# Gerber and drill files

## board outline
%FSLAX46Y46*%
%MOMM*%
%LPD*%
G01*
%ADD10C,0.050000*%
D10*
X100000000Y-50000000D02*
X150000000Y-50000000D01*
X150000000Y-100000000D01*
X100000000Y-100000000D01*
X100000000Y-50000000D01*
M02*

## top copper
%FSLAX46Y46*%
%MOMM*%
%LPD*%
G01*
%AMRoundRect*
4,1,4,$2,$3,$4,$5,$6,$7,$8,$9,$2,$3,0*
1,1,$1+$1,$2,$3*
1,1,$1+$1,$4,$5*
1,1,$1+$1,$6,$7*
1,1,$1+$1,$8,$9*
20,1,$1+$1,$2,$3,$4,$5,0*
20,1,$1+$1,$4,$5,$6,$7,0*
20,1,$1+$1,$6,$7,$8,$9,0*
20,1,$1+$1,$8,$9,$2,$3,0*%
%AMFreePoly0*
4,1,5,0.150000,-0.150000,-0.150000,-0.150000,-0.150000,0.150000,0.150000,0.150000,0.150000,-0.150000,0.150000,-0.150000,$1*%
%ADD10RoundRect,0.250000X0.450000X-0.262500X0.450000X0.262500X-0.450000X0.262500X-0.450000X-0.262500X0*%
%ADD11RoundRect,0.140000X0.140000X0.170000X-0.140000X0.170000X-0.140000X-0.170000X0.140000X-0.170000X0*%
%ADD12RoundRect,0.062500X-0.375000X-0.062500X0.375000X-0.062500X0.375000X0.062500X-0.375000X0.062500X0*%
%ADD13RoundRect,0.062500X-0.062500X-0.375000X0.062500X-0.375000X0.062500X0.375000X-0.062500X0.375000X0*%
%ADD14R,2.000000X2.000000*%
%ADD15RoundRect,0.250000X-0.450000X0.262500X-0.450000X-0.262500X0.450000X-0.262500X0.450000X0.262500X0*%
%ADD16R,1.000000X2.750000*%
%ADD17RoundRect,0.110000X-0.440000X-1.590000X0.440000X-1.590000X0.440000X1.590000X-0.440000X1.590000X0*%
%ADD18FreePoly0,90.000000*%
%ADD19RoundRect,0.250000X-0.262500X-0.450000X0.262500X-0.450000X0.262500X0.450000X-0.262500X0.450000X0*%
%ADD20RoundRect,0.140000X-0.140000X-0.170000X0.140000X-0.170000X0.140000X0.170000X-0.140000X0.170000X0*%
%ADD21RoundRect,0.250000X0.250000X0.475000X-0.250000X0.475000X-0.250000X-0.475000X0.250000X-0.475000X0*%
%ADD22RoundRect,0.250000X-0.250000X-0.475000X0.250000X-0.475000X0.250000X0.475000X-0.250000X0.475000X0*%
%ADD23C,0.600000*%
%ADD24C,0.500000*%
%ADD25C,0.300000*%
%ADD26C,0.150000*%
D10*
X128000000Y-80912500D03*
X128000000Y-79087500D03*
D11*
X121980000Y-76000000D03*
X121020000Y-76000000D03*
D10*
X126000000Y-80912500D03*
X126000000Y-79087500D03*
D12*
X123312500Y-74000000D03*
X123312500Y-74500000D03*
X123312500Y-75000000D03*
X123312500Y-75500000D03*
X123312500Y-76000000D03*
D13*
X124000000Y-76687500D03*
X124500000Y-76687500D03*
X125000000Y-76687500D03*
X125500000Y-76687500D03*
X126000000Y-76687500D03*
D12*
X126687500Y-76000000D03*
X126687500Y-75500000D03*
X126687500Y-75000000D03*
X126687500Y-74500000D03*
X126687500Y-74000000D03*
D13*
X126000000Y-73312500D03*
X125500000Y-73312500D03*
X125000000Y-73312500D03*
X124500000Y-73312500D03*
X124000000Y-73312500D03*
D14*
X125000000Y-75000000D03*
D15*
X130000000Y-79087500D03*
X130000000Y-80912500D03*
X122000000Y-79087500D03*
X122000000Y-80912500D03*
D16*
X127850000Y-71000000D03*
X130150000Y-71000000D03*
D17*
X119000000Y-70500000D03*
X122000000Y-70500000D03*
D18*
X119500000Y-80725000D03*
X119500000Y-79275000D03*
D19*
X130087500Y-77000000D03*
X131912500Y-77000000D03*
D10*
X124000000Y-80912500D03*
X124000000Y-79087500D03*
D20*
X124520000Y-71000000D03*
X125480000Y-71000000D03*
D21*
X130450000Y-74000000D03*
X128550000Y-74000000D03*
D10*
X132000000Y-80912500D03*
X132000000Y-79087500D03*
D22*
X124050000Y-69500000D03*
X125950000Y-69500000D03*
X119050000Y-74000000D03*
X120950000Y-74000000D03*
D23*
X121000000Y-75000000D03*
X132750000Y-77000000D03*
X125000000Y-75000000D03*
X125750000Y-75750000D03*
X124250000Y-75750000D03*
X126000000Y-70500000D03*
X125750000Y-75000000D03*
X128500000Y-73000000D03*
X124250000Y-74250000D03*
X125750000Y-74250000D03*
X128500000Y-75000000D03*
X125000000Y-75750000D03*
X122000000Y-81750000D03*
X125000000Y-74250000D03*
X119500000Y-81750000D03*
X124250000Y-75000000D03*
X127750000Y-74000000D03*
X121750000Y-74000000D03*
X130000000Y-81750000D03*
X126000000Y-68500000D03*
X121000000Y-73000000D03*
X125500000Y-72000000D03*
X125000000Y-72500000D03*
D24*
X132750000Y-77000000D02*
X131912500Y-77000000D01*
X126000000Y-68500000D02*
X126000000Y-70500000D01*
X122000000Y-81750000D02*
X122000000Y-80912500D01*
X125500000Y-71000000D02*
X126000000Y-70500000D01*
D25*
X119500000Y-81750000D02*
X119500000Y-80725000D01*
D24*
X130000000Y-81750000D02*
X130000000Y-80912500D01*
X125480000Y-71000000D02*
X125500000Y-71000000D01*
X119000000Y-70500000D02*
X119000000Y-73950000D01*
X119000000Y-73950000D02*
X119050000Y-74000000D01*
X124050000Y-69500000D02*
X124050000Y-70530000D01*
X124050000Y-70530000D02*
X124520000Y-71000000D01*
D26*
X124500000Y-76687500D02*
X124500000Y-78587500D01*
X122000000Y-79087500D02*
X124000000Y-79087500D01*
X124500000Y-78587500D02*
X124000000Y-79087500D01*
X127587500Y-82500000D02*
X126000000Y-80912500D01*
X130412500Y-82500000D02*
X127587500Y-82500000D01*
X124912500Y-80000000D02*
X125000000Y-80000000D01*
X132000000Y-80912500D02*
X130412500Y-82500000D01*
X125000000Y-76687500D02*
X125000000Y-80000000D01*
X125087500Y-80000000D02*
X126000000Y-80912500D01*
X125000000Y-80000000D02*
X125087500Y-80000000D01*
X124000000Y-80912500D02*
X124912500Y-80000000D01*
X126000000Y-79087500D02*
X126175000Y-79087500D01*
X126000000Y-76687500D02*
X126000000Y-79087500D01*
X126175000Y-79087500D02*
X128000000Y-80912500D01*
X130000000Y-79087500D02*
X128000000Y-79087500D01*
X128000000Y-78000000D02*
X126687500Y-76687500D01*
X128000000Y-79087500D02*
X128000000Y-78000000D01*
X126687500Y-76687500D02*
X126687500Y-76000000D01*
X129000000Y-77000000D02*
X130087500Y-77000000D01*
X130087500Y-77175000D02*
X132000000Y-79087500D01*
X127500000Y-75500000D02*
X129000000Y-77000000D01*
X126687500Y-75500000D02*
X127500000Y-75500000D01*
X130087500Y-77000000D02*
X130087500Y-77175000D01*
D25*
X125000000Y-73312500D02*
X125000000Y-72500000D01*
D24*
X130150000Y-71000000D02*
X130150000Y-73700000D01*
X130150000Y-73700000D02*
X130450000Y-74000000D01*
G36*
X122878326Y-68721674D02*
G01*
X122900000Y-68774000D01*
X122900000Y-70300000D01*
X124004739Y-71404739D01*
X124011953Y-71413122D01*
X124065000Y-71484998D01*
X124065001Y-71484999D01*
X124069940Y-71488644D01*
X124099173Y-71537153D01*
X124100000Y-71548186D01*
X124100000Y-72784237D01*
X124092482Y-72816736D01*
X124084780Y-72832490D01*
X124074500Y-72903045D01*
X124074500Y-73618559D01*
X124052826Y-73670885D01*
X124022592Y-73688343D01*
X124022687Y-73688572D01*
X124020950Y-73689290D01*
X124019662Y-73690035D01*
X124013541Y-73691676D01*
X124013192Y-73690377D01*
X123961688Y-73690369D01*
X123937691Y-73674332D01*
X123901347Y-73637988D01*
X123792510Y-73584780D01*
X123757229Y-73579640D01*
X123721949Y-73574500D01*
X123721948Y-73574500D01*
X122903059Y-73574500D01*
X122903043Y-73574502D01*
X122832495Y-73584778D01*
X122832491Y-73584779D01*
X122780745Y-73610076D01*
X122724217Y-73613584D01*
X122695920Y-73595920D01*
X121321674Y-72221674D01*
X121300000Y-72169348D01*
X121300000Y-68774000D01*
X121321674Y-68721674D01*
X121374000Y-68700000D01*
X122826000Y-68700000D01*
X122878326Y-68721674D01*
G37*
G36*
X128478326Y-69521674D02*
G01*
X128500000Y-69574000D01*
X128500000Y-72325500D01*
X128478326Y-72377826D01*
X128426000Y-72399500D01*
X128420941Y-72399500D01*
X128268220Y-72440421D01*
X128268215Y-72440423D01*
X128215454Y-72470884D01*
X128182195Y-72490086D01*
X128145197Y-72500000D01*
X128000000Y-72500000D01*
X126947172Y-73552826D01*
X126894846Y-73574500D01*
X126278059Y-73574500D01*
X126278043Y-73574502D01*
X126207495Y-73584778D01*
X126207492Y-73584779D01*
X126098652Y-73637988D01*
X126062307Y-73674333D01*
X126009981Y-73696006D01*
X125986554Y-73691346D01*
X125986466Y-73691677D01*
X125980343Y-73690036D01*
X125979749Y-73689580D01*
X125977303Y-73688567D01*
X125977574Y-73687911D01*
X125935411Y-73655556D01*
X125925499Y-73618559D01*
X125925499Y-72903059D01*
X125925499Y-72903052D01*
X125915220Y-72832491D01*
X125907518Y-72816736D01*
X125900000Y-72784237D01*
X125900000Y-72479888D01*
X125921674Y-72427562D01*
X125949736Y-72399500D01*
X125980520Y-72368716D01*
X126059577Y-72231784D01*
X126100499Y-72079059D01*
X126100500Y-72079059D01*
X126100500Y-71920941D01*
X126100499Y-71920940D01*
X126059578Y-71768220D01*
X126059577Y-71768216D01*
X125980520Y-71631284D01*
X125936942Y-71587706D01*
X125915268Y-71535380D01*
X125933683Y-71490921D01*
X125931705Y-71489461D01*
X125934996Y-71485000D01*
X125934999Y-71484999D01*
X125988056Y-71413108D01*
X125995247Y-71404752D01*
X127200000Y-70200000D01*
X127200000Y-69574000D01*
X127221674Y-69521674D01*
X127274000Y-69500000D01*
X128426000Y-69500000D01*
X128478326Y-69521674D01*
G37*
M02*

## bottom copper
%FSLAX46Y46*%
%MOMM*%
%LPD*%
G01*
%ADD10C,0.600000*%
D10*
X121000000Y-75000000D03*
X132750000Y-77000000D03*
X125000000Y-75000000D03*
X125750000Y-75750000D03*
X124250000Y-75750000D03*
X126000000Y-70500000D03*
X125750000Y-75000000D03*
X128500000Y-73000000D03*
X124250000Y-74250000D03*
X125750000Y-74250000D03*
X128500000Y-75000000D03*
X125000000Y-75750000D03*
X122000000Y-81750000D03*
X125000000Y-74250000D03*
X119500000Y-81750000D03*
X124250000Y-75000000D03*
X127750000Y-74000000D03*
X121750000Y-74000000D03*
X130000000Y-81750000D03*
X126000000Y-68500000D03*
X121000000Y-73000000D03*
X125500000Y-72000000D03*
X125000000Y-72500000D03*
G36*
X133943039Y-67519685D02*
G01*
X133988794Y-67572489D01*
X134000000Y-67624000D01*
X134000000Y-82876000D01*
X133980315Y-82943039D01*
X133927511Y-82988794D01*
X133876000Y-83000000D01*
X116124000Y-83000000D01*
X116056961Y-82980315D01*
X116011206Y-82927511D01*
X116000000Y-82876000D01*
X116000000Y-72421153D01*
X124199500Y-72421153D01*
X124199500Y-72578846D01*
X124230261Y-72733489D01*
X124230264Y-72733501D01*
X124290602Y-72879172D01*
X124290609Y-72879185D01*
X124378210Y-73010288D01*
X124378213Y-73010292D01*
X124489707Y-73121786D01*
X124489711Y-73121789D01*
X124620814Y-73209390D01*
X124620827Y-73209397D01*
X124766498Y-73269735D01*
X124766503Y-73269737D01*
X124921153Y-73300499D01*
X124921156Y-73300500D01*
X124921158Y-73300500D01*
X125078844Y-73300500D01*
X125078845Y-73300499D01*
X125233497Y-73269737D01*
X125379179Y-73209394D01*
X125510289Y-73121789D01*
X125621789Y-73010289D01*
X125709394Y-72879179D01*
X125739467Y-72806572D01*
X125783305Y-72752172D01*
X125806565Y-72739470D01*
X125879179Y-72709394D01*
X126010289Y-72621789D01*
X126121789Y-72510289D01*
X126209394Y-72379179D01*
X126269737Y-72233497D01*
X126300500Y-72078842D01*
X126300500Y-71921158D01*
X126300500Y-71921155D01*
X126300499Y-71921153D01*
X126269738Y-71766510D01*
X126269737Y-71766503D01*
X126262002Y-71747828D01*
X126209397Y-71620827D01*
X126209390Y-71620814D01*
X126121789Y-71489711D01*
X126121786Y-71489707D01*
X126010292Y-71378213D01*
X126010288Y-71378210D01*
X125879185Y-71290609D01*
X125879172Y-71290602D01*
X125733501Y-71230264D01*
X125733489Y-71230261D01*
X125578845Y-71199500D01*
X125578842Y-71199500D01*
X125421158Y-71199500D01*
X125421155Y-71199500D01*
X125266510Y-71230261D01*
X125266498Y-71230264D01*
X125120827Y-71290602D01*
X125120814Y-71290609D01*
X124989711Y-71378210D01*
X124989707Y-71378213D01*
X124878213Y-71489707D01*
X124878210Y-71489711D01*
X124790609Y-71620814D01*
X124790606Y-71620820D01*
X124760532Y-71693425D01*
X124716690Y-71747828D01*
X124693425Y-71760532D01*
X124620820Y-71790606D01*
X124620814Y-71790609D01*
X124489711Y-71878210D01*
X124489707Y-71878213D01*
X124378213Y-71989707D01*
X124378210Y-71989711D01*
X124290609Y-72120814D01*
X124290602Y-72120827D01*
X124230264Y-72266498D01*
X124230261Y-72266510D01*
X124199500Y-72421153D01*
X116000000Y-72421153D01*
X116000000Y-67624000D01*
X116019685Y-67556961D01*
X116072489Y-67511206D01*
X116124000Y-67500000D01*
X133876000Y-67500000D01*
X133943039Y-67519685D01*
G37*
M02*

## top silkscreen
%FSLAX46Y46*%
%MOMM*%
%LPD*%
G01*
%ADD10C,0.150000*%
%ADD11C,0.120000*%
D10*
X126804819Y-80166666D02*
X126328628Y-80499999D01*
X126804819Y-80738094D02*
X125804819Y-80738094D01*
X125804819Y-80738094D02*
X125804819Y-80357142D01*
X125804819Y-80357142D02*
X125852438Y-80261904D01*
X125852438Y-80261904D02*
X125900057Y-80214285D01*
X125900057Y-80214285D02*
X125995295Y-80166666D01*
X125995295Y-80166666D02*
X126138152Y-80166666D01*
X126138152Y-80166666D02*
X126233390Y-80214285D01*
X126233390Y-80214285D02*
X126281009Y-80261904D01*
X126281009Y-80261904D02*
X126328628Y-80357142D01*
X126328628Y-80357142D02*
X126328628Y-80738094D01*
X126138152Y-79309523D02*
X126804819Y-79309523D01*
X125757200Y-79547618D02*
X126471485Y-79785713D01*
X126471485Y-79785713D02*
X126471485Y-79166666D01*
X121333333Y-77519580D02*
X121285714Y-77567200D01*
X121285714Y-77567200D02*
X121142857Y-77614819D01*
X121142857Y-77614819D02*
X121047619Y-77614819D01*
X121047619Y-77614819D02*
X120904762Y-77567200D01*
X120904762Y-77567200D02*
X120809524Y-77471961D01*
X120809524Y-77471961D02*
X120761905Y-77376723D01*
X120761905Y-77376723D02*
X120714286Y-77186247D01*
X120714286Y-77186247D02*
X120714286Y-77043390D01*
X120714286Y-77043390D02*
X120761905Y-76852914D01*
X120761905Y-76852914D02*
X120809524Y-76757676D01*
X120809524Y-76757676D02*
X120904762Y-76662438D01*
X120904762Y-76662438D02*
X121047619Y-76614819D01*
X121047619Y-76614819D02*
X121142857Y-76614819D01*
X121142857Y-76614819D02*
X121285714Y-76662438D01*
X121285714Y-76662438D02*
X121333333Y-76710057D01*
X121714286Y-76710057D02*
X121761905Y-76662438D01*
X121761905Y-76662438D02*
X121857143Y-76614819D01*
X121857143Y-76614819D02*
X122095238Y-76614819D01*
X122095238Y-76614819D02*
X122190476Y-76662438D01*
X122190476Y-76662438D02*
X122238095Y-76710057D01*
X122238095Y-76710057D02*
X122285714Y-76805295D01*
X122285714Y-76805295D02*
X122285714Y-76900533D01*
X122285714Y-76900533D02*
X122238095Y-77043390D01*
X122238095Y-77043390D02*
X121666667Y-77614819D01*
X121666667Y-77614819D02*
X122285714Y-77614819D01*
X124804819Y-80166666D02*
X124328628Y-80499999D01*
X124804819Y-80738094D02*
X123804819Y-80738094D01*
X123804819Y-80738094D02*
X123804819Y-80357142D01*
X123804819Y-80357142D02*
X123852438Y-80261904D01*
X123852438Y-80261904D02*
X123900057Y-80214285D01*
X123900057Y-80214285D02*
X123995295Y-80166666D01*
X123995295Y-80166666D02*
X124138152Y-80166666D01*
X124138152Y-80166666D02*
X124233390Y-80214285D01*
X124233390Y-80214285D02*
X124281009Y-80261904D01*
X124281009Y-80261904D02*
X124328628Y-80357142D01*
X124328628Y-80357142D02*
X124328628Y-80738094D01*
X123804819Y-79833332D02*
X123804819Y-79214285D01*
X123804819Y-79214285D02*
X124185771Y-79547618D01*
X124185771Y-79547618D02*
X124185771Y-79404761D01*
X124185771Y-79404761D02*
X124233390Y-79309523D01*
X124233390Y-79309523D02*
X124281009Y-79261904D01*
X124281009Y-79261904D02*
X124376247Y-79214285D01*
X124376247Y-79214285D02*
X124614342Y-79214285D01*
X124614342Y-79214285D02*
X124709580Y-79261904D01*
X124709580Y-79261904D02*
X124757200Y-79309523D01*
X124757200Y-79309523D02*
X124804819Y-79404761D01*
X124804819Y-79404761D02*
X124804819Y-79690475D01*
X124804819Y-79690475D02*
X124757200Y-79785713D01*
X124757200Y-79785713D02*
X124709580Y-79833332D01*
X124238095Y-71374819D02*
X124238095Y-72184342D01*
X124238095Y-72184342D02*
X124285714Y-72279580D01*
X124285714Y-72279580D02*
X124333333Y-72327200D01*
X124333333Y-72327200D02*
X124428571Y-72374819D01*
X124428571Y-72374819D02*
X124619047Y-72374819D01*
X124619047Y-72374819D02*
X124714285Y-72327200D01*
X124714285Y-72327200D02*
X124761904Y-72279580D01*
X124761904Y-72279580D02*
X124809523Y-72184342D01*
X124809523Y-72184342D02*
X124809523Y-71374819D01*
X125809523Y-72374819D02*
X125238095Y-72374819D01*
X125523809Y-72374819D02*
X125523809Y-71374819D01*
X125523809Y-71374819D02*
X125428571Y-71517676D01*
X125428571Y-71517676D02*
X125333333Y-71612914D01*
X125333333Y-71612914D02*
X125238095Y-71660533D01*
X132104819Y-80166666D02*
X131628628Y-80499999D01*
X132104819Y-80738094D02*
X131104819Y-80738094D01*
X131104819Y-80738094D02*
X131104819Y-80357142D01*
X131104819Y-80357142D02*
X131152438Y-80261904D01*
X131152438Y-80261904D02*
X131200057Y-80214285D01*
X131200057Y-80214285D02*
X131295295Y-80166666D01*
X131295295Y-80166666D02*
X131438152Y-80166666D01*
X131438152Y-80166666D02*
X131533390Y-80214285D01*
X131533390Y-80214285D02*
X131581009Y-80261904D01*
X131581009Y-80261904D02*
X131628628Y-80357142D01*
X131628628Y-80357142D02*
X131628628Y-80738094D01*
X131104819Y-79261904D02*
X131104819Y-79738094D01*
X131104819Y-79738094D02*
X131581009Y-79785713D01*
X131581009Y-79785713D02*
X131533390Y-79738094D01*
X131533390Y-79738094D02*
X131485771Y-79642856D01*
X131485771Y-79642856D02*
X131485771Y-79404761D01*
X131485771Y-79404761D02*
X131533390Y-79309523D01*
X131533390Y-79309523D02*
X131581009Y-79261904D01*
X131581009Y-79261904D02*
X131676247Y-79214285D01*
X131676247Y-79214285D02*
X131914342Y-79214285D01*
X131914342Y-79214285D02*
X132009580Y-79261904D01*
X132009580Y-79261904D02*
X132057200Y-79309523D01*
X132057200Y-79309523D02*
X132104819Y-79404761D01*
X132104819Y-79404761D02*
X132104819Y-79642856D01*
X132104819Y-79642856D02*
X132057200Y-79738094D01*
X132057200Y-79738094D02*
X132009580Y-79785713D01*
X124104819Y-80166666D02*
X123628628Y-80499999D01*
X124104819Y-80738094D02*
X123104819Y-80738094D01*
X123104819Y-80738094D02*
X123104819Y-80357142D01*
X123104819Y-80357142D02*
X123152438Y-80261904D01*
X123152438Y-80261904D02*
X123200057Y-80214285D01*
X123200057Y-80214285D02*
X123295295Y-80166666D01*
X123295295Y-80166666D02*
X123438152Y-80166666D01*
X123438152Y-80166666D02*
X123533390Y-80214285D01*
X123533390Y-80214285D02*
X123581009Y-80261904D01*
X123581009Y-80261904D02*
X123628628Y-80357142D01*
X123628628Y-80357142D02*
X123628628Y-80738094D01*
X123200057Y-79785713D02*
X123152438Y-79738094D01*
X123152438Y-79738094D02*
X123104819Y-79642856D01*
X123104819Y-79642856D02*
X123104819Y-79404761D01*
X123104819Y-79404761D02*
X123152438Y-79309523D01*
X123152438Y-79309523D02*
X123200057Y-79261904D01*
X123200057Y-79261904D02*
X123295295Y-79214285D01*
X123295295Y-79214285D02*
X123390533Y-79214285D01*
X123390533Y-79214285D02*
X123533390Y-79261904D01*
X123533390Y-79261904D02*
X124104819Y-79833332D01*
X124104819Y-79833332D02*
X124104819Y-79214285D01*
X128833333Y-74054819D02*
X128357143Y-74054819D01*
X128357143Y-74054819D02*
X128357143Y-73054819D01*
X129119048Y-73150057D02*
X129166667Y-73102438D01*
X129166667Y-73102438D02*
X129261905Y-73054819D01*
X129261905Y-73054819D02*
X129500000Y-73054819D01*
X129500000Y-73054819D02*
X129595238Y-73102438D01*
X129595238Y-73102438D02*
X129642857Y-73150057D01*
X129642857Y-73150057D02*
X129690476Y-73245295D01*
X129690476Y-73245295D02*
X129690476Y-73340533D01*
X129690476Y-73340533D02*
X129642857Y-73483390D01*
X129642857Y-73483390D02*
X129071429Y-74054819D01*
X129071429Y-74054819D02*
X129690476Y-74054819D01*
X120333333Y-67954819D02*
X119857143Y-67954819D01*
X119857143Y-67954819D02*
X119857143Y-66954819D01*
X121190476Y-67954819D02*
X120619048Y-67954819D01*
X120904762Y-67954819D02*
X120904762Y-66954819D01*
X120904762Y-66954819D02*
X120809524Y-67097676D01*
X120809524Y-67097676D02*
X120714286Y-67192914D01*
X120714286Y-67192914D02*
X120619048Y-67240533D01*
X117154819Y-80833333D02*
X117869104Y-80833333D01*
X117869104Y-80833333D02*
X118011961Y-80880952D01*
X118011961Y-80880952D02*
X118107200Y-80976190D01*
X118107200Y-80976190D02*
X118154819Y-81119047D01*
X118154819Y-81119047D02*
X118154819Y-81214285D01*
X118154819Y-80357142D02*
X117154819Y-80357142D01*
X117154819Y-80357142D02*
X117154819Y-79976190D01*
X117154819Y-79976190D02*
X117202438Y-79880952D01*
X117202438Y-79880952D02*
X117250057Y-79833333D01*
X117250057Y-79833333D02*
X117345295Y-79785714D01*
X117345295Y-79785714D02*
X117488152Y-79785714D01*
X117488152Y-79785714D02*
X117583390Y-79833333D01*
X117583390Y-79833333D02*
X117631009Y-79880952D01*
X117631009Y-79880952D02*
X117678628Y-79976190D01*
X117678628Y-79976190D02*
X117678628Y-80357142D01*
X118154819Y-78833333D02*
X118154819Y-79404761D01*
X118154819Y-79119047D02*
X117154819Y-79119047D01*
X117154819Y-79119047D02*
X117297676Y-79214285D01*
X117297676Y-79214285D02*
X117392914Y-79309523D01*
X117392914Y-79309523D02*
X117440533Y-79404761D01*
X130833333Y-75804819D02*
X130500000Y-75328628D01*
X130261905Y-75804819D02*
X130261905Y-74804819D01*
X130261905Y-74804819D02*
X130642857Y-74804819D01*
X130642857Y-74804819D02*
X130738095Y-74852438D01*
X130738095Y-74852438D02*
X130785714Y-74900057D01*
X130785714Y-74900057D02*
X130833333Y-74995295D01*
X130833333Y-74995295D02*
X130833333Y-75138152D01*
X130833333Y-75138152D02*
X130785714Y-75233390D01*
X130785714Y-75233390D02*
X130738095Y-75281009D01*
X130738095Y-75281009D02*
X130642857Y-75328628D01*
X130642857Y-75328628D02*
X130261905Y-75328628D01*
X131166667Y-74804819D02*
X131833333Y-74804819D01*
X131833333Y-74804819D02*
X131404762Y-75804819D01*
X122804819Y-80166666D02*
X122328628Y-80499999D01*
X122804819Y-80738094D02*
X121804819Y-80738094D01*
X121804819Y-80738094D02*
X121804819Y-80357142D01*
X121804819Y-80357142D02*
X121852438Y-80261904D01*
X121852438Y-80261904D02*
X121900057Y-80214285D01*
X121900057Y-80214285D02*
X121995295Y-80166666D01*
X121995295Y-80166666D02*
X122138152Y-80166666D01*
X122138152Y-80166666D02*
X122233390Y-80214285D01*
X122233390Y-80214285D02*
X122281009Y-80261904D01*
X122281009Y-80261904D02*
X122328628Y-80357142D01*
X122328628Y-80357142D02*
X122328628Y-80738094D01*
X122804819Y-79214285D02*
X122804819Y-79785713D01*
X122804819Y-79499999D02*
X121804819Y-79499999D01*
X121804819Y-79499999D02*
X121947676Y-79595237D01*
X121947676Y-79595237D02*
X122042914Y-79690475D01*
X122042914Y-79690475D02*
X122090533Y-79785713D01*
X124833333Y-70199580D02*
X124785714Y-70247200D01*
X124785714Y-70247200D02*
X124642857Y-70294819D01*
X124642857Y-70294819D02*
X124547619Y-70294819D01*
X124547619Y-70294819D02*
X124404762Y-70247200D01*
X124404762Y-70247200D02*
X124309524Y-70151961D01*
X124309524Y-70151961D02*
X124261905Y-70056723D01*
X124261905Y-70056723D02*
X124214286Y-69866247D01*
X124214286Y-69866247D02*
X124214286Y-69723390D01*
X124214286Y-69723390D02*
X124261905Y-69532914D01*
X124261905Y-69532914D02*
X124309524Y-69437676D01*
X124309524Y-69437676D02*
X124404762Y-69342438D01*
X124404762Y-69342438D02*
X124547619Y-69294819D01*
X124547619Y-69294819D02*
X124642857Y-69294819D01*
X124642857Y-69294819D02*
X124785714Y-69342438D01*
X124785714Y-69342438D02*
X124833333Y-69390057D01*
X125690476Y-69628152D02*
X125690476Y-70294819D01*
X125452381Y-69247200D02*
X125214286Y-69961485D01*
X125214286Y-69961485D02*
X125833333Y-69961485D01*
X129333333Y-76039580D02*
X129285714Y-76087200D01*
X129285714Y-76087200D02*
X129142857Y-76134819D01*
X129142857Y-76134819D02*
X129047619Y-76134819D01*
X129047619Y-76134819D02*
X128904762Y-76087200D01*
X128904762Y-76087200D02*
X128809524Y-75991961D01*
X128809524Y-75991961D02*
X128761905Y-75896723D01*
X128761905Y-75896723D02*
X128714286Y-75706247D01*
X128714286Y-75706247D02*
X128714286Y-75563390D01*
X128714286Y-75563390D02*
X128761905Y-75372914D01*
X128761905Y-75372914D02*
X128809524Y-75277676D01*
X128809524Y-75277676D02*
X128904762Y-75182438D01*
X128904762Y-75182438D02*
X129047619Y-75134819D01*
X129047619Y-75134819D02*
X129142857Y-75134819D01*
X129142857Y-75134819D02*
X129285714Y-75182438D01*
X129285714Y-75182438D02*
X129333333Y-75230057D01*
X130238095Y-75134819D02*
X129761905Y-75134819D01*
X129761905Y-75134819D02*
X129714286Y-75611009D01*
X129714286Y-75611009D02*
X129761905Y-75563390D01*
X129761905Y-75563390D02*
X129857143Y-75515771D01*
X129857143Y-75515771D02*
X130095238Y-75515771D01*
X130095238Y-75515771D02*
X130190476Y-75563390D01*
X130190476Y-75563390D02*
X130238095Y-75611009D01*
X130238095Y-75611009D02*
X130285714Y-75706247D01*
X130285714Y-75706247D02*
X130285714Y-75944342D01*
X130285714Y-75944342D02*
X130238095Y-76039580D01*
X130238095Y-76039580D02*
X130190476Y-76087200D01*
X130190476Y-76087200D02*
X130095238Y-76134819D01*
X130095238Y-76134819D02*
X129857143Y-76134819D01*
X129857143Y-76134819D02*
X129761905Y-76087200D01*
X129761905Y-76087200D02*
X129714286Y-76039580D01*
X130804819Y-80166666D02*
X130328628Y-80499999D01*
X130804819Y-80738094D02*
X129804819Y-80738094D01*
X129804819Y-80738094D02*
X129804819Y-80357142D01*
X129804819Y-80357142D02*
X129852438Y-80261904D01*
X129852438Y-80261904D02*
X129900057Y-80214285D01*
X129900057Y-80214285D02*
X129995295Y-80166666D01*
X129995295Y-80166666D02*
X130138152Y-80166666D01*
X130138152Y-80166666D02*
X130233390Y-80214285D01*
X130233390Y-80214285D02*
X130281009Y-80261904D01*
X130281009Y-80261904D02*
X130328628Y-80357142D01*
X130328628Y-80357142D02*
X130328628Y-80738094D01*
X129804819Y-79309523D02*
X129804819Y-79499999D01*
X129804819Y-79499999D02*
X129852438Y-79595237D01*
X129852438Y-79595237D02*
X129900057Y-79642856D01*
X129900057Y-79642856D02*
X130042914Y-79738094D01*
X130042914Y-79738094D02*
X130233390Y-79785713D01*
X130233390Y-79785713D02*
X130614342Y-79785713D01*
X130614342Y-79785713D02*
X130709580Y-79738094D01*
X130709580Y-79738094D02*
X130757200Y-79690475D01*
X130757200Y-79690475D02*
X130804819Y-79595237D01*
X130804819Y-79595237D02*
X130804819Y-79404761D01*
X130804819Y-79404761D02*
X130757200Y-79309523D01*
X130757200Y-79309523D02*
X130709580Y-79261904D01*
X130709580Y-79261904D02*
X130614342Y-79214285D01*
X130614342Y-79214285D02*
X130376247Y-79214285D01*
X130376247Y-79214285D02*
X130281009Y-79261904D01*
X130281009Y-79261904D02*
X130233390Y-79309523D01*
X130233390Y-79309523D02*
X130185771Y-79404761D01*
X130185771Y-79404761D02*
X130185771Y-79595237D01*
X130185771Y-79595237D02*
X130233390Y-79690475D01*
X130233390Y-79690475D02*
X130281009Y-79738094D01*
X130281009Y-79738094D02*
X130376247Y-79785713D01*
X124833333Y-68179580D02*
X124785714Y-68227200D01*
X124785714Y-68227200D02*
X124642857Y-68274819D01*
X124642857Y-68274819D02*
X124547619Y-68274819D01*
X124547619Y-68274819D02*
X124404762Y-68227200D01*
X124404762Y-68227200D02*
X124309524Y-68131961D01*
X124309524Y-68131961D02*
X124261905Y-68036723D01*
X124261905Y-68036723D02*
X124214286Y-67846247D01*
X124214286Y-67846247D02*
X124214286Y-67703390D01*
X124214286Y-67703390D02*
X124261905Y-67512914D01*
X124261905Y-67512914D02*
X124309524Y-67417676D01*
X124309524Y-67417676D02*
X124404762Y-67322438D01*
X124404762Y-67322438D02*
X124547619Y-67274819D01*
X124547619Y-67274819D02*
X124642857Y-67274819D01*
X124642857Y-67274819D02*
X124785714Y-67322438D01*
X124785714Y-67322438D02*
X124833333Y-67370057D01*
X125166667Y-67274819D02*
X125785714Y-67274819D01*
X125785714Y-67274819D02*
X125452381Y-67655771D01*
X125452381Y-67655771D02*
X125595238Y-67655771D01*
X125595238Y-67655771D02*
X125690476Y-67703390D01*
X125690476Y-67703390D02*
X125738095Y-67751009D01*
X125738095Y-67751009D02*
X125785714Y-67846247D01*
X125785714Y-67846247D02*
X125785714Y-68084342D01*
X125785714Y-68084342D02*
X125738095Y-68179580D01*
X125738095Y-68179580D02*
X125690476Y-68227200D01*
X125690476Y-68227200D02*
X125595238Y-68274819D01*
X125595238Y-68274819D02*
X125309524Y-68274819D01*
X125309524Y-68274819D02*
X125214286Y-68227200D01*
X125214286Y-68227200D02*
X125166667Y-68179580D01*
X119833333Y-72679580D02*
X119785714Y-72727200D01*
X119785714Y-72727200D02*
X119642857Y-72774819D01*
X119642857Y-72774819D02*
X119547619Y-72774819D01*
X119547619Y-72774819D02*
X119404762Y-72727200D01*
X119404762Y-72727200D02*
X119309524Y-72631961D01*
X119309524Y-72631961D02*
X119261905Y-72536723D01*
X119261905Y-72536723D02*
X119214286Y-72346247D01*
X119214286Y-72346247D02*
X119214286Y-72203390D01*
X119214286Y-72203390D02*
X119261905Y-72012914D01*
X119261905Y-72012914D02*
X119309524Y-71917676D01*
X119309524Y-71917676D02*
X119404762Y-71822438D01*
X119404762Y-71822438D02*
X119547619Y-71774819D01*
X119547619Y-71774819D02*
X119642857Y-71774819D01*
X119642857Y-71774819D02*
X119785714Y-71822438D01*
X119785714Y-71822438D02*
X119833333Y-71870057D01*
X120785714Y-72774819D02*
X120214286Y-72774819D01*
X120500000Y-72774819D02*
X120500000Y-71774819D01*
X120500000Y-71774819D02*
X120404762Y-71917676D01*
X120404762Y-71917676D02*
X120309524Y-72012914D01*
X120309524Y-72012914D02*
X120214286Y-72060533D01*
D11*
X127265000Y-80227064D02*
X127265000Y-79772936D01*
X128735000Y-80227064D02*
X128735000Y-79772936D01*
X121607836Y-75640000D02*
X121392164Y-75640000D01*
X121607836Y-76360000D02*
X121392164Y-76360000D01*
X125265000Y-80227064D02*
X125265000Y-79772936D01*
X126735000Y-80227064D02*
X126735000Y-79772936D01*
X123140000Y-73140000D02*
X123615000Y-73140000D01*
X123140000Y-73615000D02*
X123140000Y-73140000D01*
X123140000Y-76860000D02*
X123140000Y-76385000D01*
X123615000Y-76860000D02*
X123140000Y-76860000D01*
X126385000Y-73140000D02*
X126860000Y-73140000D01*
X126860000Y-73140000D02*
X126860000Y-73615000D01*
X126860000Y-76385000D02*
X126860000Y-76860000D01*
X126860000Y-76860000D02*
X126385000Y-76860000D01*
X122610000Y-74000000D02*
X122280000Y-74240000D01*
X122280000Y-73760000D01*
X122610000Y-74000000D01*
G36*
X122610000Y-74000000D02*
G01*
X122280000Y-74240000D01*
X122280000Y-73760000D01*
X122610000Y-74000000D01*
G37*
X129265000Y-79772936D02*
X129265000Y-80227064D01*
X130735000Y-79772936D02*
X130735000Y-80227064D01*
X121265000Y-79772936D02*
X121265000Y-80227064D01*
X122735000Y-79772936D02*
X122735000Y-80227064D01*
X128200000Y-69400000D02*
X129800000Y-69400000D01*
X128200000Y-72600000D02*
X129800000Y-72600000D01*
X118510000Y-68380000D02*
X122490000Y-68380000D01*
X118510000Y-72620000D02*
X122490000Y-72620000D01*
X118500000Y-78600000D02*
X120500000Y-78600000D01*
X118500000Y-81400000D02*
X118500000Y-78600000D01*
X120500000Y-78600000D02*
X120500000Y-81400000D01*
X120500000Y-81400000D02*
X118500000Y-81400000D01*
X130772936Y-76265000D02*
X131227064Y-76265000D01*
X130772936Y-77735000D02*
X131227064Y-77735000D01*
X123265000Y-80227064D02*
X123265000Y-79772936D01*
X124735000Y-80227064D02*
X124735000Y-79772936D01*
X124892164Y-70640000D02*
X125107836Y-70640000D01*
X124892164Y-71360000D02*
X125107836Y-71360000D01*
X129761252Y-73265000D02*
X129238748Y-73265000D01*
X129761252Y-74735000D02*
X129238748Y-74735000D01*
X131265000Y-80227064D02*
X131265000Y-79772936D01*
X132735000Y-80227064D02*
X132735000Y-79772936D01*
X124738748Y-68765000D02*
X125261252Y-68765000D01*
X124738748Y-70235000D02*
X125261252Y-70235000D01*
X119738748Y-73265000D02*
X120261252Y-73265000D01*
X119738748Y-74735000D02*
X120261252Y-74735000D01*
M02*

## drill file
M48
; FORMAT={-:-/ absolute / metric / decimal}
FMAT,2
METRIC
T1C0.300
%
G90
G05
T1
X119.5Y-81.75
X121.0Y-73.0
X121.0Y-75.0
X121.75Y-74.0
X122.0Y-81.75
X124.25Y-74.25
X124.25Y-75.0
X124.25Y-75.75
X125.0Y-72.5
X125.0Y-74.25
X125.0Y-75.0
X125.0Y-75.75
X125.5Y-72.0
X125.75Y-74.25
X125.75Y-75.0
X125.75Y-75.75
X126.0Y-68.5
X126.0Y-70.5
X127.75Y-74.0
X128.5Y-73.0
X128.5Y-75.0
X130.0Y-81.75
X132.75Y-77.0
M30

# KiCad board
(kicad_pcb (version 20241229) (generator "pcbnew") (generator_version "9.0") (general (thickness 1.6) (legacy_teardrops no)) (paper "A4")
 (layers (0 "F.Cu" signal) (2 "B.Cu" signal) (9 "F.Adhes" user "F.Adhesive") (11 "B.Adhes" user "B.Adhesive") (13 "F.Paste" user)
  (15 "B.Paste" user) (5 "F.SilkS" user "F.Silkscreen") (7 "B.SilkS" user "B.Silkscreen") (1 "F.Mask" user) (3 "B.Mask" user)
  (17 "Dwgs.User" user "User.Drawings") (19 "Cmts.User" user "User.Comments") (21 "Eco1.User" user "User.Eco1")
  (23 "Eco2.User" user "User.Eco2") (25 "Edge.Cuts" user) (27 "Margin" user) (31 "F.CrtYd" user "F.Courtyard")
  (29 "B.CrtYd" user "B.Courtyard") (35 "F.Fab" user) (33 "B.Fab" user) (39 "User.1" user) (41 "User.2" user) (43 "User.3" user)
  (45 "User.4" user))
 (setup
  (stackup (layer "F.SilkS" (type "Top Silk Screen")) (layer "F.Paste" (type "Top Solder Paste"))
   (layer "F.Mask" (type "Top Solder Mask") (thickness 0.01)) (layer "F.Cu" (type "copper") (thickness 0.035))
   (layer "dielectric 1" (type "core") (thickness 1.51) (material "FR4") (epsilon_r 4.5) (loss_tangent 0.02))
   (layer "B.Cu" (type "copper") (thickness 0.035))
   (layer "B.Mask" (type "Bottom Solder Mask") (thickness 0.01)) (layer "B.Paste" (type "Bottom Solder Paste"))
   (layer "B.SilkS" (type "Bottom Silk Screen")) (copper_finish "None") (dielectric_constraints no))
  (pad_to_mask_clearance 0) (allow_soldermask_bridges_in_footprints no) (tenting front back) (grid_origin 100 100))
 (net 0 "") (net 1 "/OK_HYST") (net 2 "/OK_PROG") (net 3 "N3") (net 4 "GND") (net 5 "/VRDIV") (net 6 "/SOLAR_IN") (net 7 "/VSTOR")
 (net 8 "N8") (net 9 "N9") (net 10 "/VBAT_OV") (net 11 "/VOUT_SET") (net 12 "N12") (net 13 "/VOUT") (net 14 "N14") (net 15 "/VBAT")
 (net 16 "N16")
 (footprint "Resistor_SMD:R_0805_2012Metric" (layer "F.Cu") (at 128 80 90)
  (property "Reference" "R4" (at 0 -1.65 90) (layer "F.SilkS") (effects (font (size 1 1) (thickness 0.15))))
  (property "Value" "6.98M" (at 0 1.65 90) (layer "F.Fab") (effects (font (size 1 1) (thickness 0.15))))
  (fp_line (start -0.227064 -0.735) (end 0.227064 -0.735) (stroke (width 0.12) (type solid)) (layer "F.SilkS"))
  (fp_line (start -0.227064 0.735) (end 0.227064 0.735) (stroke (width 0.12) (type solid)) (layer "F.SilkS"))
  (pad "1" smd roundrect (at -0.9125 0 90) (size 1.025 1.4) (layers "F.Cu" "F.Mask" "F.Paste") (roundrect_rratio 0.243902)
   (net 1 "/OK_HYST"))
  (pad "2" smd roundrect (at 0.9125 0 90) (size 1.025 1.4) (layers "F.Cu" "F.Mask" "F.Paste") (roundrect_rratio 0.243902) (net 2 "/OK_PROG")))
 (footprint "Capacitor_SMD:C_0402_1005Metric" (layer "F.Cu") (at 121.5 76 180)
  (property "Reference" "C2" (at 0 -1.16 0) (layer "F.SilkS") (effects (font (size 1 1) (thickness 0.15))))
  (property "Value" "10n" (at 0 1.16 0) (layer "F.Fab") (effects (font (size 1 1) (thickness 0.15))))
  (fp_line (start -0.107836 0.36) (end 0.107836 0.36) (stroke (width 0.12) (type solid)) (layer "F.SilkS"))
  (fp_line (start -0.107836 -0.36) (end 0.107836 -0.36) (stroke (width 0.12) (type solid)) (layer "F.SilkS"))
  (pad "1" smd roundrect (at -0.48 0 180) (size 0.56 0.62) (layers "F.Cu" "F.Mask" "F.Paste") (roundrect_rratio 0.25) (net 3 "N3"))
  (pad "2" smd roundrect (at 0.48 0 180) (size 0.56 0.62) (layers "F.Cu" "F.Mask" "F.Paste") (roundrect_rratio 0.25) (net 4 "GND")))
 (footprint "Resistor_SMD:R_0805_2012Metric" (layer "F.Cu") (at 126 80 90)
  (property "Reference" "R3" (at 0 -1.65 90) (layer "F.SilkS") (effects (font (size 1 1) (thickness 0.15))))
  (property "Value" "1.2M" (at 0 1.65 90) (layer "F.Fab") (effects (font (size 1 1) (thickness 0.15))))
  (fp_line (start -0.227064 -0.735) (end 0.227064 -0.735) (stroke (width 0.12) (type solid)) (layer "F.SilkS"))
  (fp_line (start -0.227064 0.735) (end 0.227064 0.735) (stroke (width 0.12) (type solid)) (layer "F.SilkS"))
  (pad "1" smd roundrect (at -0.9125 0 90) (size 1.025 1.4) (layers "F.Cu" "F.Mask" "F.Paste") (roundrect_rratio 0.243902) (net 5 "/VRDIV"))
  (pad "2" smd roundrect (at 0.9125 0 90) (size 1.025 1.4) (layers "F.Cu" "F.Mask" "F.Paste") (roundrect_rratio 0.243902) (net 1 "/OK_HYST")))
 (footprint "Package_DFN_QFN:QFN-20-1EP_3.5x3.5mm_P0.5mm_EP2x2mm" (layer "F.Cu") (at 125 75)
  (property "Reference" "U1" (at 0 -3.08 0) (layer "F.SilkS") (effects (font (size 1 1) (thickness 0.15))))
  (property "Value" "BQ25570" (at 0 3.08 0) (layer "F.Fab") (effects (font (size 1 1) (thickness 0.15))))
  (fp_line (start -1.86 -1.86) (end -1.385 -1.86) (stroke (width 0.12) (type solid)) (layer "F.SilkS"))
  (fp_line (start -1.86 -1.385) (end -1.86 -1.86) (stroke (width 0.12) (type solid)) (layer "F.SilkS"))
  (fp_line (start -1.86 1.86) (end -1.86 1.385) (stroke (width 0.12) (type solid)) (layer "F.SilkS"))
  (fp_line (start -1.385 1.86) (end -1.86 1.86) (stroke (width 0.12) (type solid)) (layer "F.SilkS"))
  (fp_line (start 1.385 -1.86) (end 1.86 -1.86) (stroke (width 0.12) (type solid)) (layer "F.SilkS"))
  (fp_line (start 1.86 -1.86) (end 1.86 -1.385) (stroke (width 0.12) (type solid)) (layer "F.SilkS"))
  (fp_line (start 1.86 1.385) (end 1.86 1.86) (stroke (width 0.12) (type solid)) (layer "F.SilkS"))
  (fp_line (start 1.86 1.86) (end 1.385 1.86) (stroke (width 0.12) (type solid)) (layer "F.SilkS"))
  (fp_poly (pts (xy -2.39 -1) (xy -2.72 -0.76) (xy -2.72 -1.24)) (stroke (width 0.12) (type solid)) (fill yes) (layer "F.SilkS"))
  (pad "" smd roundrect (at -0.5 -0.5) (size 0.81 0.81) (layers "F.Paste") (roundrect_rratio 0.25))
  (pad "" smd roundrect (at -0.5 0.5) (size 0.81 0.81) (layers "F.Paste") (roundrect_rratio 0.25))
  (pad "" smd roundrect (at 0.5 -0.5) (size 0.81 0.81) (layers "F.Paste") (roundrect_rratio 0.25))
  (pad "" smd roundrect (at 0.5 0.5) (size 0.81 0.81) (layers "F.Paste") (roundrect_rratio 0.25))
  (pad "1" smd roundrect (at -1.6875 -1) (size 0.875 0.25) (layers "F.Cu" "F.Mask" "F.Paste") (roundrect_rratio 0.25) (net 4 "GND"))
  (pad "2" smd roundrect (at -1.6875 -0.5) (size 0.875 0.25) (layers "F.Cu" "F.Mask" "F.Paste") (roundrect_rratio 0.25) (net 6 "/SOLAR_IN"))
  (pad "3" smd roundrect (at -1.6875 0) (size 0.875 0.25) (layers "F.Cu" "F.Mask" "F.Paste") (roundrect_rratio 0.25) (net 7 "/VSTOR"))
  (pad "4" smd roundrect (at -1.6875 0.5) (size 0.875 0.25) (layers "F.Cu" "F.Mask" "F.Paste") (roundrect_rratio 0.25) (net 3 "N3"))
  (pad "5" smd roundrect (at -1.6875 1) (size 0.875 0.25) (layers "F.Cu" "F.Mask" "F.Paste") (roundrect_rratio 0.25) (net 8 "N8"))
  (pad "6" smd roundrect (at -1 1.6875) (size 0.25 0.875) (layers "F.Cu" "F.Mask" "F.Paste") (roundrect_rratio 0.25) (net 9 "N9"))
  (pad "7" smd roundrect (at -0.5 1.6875) (size 0.25 0.875) (layers "F.Cu" "F.Mask" "F.Paste") (roundrect_rratio 0.25) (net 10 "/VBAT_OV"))
  (pad "8" smd roundrect (at 0 1.6875) (size 0.25 0.875) (layers "F.Cu" "F.Mask" "F.Paste") (roundrect_rratio 0.25) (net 5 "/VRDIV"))
  (pad "9" smd roundrect (at 0.5 1.6875) (size 0.25 0.875) (layers "F.Cu" "F.Mask" "F.Paste") (roundrect_rratio 0.25) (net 4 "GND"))
  (pad "10" smd roundrect (at 1 1.6875) (size 0.25 0.875) (layers "F.Cu" "F.Mask" "F.Paste") (roundrect_rratio 0.25) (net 1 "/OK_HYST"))
  (pad "11" smd roundrect (at 1.6875 1) (size 0.875 0.25) (layers "F.Cu" "F.Mask" "F.Paste") (roundrect_rratio 0.25) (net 2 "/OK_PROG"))
  (pad "12" smd roundrect (at 1.6875 0.5) (size 0.875 0.25) (layers "F.Cu" "F.Mask" "F.Paste") (roundrect_rratio 0.25) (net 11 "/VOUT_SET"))
  (pad "13" smd roundrect (at 1.6875 0) (size 0.875 0.25) (layers "F.Cu" "F.Mask" "F.Paste") (roundrect_rratio 0.25) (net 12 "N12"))
  (pad "14" smd roundrect (at 1.6875 -0.5) (size 0.875 0.25) (layers "F.Cu" "F.Mask" "F.Paste") (roundrect_rratio 0.25) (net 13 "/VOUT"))
  (pad "15" smd roundrect (at 1.6875 -1) (size 0.875 0.25) (layers "F.Cu" "F.Mask" "F.Paste") (roundrect_rratio 0.25) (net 4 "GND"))
  (pad "16" smd roundrect (at 1 -1.6875) (size 0.25 0.875) (layers "F.Cu" "F.Mask" "F.Paste") (roundrect_rratio 0.25) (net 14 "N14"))
  (pad "17" smd roundrect (at 0.5 -1.6875) (size 0.25 0.875) (layers "F.Cu" "F.Mask" "F.Paste") (roundrect_rratio 0.25) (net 4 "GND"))
  (pad "18" smd roundrect (at 0 -1.6875) (size 0.25 0.875) (layers "F.Cu" "F.Mask" "F.Paste") (roundrect_rratio 0.25) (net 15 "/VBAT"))
  (pad "19" smd roundrect (at -0.5 -1.6875) (size 0.25 0.875) (layers "F.Cu" "F.Mask" "F.Paste") (roundrect_rratio 0.25) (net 7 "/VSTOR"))
  (pad "20" smd roundrect (at -1 -1.6875) (size 0.25 0.875) (layers "F.Cu" "F.Mask" "F.Paste") (roundrect_rratio 0.25) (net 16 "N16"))
  (pad "21" smd rect (at 0 0) (size 2 2) (layers "F.Cu" "F.Mask") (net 4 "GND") (zone_connect 2)))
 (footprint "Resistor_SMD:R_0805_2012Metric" (layer "F.Cu") (at 130 80 -90)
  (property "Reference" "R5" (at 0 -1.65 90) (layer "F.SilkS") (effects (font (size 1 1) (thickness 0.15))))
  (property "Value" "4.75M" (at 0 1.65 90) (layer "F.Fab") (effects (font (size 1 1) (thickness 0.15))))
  (fp_line (start -0.227064 0.735) (end 0.227064 0.735) (stroke (width 0.12) (type solid)) (layer "F.SilkS"))
  (fp_line (start -0.227064 -0.735) (end 0.227064 -0.735) (stroke (width 0.12) (type solid)) (layer "F.SilkS"))
  (pad "1" smd roundrect (at -0.9125 0 270) (size 1.025 1.4) (layers "F.Cu" "F.Mask" "F.Paste") (roundrect_rratio 0.243902)
   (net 2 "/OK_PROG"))
  (pad "2" smd roundrect (at 0.9125 0 270) (size 1.025 1.4) (layers "F.Cu" "F.Mask" "F.Paste") (roundrect_rratio 0.243902) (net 4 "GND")))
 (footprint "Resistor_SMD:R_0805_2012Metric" (layer "F.Cu") (at 122 80 -90)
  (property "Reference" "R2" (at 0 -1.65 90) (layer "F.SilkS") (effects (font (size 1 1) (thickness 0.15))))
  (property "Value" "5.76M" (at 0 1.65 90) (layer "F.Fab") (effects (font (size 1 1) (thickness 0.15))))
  (fp_line (start -0.227064 0.735) (end 0.227064 0.735) (stroke (width 0.12) (type solid)) (layer "F.SilkS"))
  (fp_line (start -0.227064 -0.735) (end 0.227064 -0.735) (stroke (width 0.12) (type solid)) (layer "F.SilkS"))
  (pad "1" smd roundrect (at -0.9125 0 270) (size 1.025 1.4) (layers "F.Cu" "F.Mask" "F.Paste") (roundrect_rratio 0.243902)
   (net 10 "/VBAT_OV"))
  (pad "2" smd roundrect (at 0.9125 0 270) (size 1.025 1.4) (layers "F.Cu" "F.Mask" "F.Paste") (roundrect_rratio 0.243902) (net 4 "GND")))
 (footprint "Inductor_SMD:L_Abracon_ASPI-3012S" (layer "F.Cu") (at 129 71)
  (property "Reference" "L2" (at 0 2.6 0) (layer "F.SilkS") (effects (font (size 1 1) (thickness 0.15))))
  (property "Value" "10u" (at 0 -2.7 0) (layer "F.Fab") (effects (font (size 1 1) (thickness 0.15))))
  (fp_line (start -0.8 -1.6) (end 0.8 -1.6) (stroke (width 0.12) (type solid)) (layer "F.SilkS"))
  (fp_line (start -0.8 1.6) (end 0.8 1.6) (stroke (width 0.12) (type solid)) (layer "F.SilkS"))
  (pad "1" smd rect (at -1.15 0) (size 1 2.75) (layers "F.Cu" "F.Mask" "F.Paste") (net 14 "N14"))
  (pad "2" smd rect (at 1.15 0) (size 1 2.75) (layers "F.Cu" "F.Mask" "F.Paste") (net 13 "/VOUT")))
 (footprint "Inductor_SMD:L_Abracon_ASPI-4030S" (layer "F.Cu") (at 120.5 70.5)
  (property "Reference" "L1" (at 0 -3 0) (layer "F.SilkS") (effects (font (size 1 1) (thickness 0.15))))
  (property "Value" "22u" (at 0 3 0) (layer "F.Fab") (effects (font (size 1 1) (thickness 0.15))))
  (fp_line (start -1.99 -2.12) (end 1.99 -2.12) (stroke (width 0.12) (type solid)) (layer "F.SilkS"))
  (fp_line (start -1.99 2.12) (end 1.99 2.12) (stroke (width 0.12) (type solid)) (layer "F.SilkS"))
  (pad "1" smd roundrect (at -1.5 0) (size 1.1 3.4) (layers "F.Cu" "F.Mask" "F.Paste") (roundrect_rratio 0.1) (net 6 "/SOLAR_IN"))
  (pad "2" smd roundrect (at 1.5 0) (size 1.1 3.4) (layers "F.Cu" "F.Mask" "F.Paste") (roundrect_rratio 0.1) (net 16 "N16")))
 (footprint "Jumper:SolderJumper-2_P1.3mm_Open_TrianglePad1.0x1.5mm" (layer "F.Cu") (at 119.5 80 90)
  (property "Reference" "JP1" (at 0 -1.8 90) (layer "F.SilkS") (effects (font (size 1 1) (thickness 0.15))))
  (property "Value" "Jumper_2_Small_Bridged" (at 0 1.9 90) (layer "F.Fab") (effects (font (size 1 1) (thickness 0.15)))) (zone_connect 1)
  (fp_line (start 1.4 -1) (end 1.4 1) (stroke (width 0.12) (type solid)) (layer "F.SilkS"))
  (fp_line (start -1.4 -1) (end 1.4 -1) (stroke (width 0.12) (type solid)) (layer "F.SilkS"))
  (fp_line (start 1.4 1) (end -1.4 1) (stroke (width 0.12) (type solid)) (layer "F.SilkS"))
  (fp_line (start -1.4 1) (end -1.4 -1) (stroke (width 0.12) (type solid)) (layer "F.SilkS"))
  (pad "1" smd custom (at -0.725 0 90) (size 0.3 0.3) (layers "F.Cu" "F.Mask") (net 4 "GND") (zone_connect 2) (thermal_bridge_angle 45)
   (options (clearance outline) (anchor rect)) (primitives))
  (pad "2" smd custom (at 0.725 0 90) (size 0.3 0.3) (layers "F.Cu" "F.Mask") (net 8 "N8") (zone_connect 2) (thermal_bridge_angle 45)
   (options (clearance outline) (anchor rect)) (primitives)))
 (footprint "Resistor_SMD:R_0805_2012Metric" (layer "F.Cu") (at 131 77)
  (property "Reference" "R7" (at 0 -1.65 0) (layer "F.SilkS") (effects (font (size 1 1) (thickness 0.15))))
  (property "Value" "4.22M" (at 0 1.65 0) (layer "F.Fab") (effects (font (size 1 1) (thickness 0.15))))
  (fp_line (start -0.227064 -0.735) (end 0.227064 -0.735) (stroke (width 0.12) (type solid)) (layer "F.SilkS"))
  (fp_line (start -0.227064 0.735) (end 0.227064 0.735) (stroke (width 0.12) (type solid)) (layer "F.SilkS"))
  (pad "1" smd roundrect (at -0.9125 0) (size 1.025 1.4) (layers "F.Cu" "F.Mask" "F.Paste") (roundrect_rratio 0.243902) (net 11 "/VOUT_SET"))
  (pad "2" smd roundrect (at 0.9125 0) (size 1.025 1.4) (layers "F.Cu" "F.Mask" "F.Paste") (roundrect_rratio 0.243902) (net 4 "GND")))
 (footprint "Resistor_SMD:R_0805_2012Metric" (layer "F.Cu") (at 124 80 90)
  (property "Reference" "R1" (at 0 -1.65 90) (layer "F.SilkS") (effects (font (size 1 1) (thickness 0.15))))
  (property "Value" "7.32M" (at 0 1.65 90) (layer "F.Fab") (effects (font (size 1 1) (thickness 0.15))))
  (fp_line (start -0.227064 -0.735) (end 0.227064 -0.735) (stroke (width 0.12) (type solid)) (layer "F.SilkS"))
  (fp_line (start -0.227064 0.735) (end 0.227064 0.735) (stroke (width 0.12) (type solid)) (layer "F.SilkS"))
  (pad "1" smd roundrect (at -0.9125 0 90) (size 1.025 1.4) (layers "F.Cu" "F.Mask" "F.Paste") (roundrect_rratio 0.243902) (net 5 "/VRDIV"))
  (pad "2" smd roundrect (at 0.9125 0 90) (size 1.025 1.4) (layers "F.Cu" "F.Mask" "F.Paste") (roundrect_rratio 0.243902)
   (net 10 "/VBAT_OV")))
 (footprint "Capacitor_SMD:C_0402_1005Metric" (layer "F.Cu") (at 125 71)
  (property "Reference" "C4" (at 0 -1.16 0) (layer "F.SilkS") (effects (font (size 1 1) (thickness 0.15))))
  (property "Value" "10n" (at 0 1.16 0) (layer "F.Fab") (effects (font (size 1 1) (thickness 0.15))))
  (fp_line (start -0.107836 -0.36) (end 0.107836 -0.36) (stroke (width 0.12) (type solid)) (layer "F.SilkS"))
  (fp_line (start -0.107836 0.36) (end 0.107836 0.36) (stroke (width 0.12) (type solid)) (layer "F.SilkS"))
  (pad "1" smd roundrect (at -0.48 0) (size 0.56 0.62) (layers "F.Cu" "F.Mask" "F.Paste") (roundrect_rratio 0.25) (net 7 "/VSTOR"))
  (pad "2" smd roundrect (at 0.48 0) (size 0.56 0.62) (layers "F.Cu" "F.Mask" "F.Paste") (roundrect_rratio 0.25) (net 4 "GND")))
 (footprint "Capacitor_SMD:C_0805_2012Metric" (layer "F.Cu") (at 129.5 74 180)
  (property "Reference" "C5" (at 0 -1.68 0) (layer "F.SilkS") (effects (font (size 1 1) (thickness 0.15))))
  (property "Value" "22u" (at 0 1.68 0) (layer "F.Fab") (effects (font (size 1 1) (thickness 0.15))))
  (fp_line (start -0.261252 0.735) (end 0.261252 0.735) (stroke (width 0.12) (type solid)) (layer "F.SilkS"))
  (fp_line (start -0.261252 -0.735) (end 0.261252 -0.735) (stroke (width 0.12) (type solid)) (layer "F.SilkS"))
  (pad "1" smd roundrect (at -0.95 0 180) (size 1 1.45) (layers "F.Cu" "F.Mask" "F.Paste") (roundrect_rratio 0.25) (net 13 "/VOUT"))
  (pad "2" smd roundrect (at 0.95 0 180) (size 1 1.45) (layers "F.Cu" "F.Mask" "F.Paste") (roundrect_rratio 0.25) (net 4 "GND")))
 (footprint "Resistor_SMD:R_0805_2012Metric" (layer "F.Cu") (at 132 80 90)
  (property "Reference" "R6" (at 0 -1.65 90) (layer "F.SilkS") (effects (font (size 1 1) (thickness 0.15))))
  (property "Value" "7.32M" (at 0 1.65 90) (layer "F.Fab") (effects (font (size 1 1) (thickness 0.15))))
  (fp_line (start -0.227064 -0.735) (end 0.227064 -0.735) (stroke (width 0.12) (type solid)) (layer "F.SilkS"))
  (fp_line (start -0.227064 0.735) (end 0.227064 0.735) (stroke (width 0.12) (type solid)) (layer "F.SilkS"))
  (pad "1" smd roundrect (at -0.9125 0 90) (size 1.025 1.4) (layers "F.Cu" "F.Mask" "F.Paste") (roundrect_rratio 0.243902) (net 5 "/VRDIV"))
  (pad "2" smd roundrect (at 0.9125 0 90) (size 1.025 1.4) (layers "F.Cu" "F.Mask" "F.Paste") (roundrect_rratio 0.243902)
   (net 11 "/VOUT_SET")))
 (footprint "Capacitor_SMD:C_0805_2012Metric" (layer "F.Cu") (at 125 69.5)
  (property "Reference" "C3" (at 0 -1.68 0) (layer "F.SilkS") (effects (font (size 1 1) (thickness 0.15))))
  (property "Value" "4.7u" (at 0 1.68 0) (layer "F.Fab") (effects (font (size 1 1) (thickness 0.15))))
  (fp_line (start -0.261252 -0.735) (end 0.261252 -0.735) (stroke (width 0.12) (type solid)) (layer "F.SilkS"))
  (fp_line (start -0.261252 0.735) (end 0.261252 0.735) (stroke (width 0.12) (type solid)) (layer "F.SilkS"))
  (pad "1" smd roundrect (at -0.95 0) (size 1 1.45) (layers "F.Cu" "F.Mask" "F.Paste") (roundrect_rratio 0.25) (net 7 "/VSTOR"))
  (pad "2" smd roundrect (at 0.95 0) (size 1 1.45) (layers "F.Cu" "F.Mask" "F.Paste") (roundrect_rratio 0.25) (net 4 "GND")))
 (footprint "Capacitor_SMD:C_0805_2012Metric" (layer "F.Cu") (at 120 74)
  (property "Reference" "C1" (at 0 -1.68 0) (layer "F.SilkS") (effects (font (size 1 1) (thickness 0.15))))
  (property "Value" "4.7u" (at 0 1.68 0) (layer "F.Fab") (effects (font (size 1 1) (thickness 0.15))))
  (fp_line (start -0.261252 -0.735) (end 0.261252 -0.735) (stroke (width 0.12) (type solid)) (layer "F.SilkS"))
  (fp_line (start -0.261252 0.735) (end 0.261252 0.735) (stroke (width 0.12) (type solid)) (layer "F.SilkS"))
  (pad "1" smd roundrect (at -0.95 0) (size 1 1.45) (layers "F.Cu" "F.Mask" "F.Paste") (roundrect_rratio 0.25) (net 6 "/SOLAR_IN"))
  (pad "2" smd roundrect (at 0.95 0) (size 1 1.45) (layers "F.Cu" "F.Mask" "F.Paste") (roundrect_rratio 0.25) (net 4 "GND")))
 (gr_rect (start 100 50) (end 150 100) (stroke (width 0.05) (type default)) (fill no) (layer "Edge.Cuts"))
 (segment (start 132.75 77) (end 131.9125 77) (width 0.5) (layer "F.Cu") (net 4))
 (segment (start 126 68.5) (end 126 70.5) (width 0.5) (layer "F.Cu") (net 4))
 (segment (start 122 81.75) (end 122 80.9125) (width 0.5) (layer "F.Cu") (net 4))
 (segment (start 125.5 71) (end 126 70.5) (width 0.5) (layer "F.Cu") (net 4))
 (segment (start 119.5 81.75) (end 119.5 80.725) (width 0.3) (layer "F.Cu") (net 4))
 (segment (start 130 81.75) (end 130 80.9125) (width 0.5) (layer "F.Cu") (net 4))
 (segment (start 125.48 71) (end 125.5 71) (width 0.5) (layer "F.Cu") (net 4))
 (via (at 121 75) (size 0.6) (drill 0.3) (layers "F.Cu" "B.Cu") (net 4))
 (via (at 132.75 77) (size 0.6) (drill 0.3) (layers "F.Cu" "B.Cu") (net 4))
 (via (at 125 75) (size 0.6) (drill 0.3) (layers "F.Cu" "B.Cu") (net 4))
 (via (at 125.75 75.75) (size 0.6) (drill 0.3) (layers "F.Cu" "B.Cu") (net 4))
 (via (at 124.25 75.75) (size 0.6) (drill 0.3) (layers "F.Cu" "B.Cu") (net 4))
 (via (at 126 70.5) (size 0.6) (drill 0.3) (layers "F.Cu" "B.Cu") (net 4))
 (via (at 125.75 75) (size 0.6) (drill 0.3) (layers "F.Cu" "B.Cu") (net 4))
 (via (at 128.5 73) (size 0.6) (drill 0.3) (layers "F.Cu" "B.Cu") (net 4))
 (via (at 124.25 74.25) (size 0.6) (drill 0.3) (layers "F.Cu" "B.Cu") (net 4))
 (via (at 125.75 74.25) (size 0.6) (drill 0.3) (layers "F.Cu" "B.Cu") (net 4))
 (via (at 128.5 75) (size 0.6) (drill 0.3) (layers "F.Cu" "B.Cu") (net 4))
 (via (at 125 75.75) (size 0.6) (drill 0.3) (layers "F.Cu" "B.Cu") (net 4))
 (via (at 122 81.75) (size 0.6) (drill 0.3) (layers "F.Cu" "B.Cu") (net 4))
 (via (at 125 74.25) (size 0.6) (drill 0.3) (layers "F.Cu" "B.Cu") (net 4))
 (via (at 119.5 81.75) (size 0.6) (drill 0.3) (layers "F.Cu" "B.Cu") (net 4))
 (via (at 124.25 75) (size 0.6) (drill 0.3) (layers "F.Cu" "B.Cu") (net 4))
 (via (at 127.75 74) (size 0.6) (drill 0.3) (layers "F.Cu" "B.Cu") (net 4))
 (via (at 121.75 74) (size 0.6) (drill 0.3) (layers "F.Cu" "B.Cu") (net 4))
 (via (at 130 81.75) (size 0.6) (drill 0.3) (layers "F.Cu" "B.Cu") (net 4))
 (via (at 126 68.5) (size 0.6) (drill 0.3) (layers "F.Cu" "B.Cu") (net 4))
 (via (at 121 73) (size 0.6) (drill 0.3) (layers "F.Cu" "B.Cu") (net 4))
 (segment (start 119 70.5) (end 119 73.95) (width 0.5) (layer "F.Cu") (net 6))
 (segment (start 119 73.95) (end 119.05 74) (width 0.5) (layer "F.Cu") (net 6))
 (segment (start 124.05 69.5) (end 124.05 70.53) (width 0.5) (layer "F.Cu") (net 7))
 (segment (start 124.05 70.53) (end 124.52 71) (width 0.5) (layer "F.Cu") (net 7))
 (segment (start 124.5 76.6875) (end 124.5 78.5875) (width 0.15) (layer "F.Cu") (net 10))
 (segment (start 122 79.0875) (end 124 79.0875) (width 0.15) (layer "F.Cu") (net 10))
 (segment (start 124.5 78.5875) (end 124 79.0875) (width 0.15) (layer "F.Cu") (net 10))
 (segment (start 127.5875 82.5) (end 126 80.9125) (width 0.15) (layer "F.Cu") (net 5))
 (segment (start 130.4125 82.5) (end 127.5875 82.5) (width 0.15) (layer "F.Cu") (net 5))
 (segment (start 124.9125 80) (end 125 80) (width 0.15) (layer "F.Cu") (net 5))
 (segment (start 132 80.9125) (end 130.4125 82.5) (width 0.15) (layer "F.Cu") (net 5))
 (segment (start 125 76.6875) (end 125 80) (width 0.15) (layer "F.Cu") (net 5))
 (segment (start 125.0875 80) (end 126 80.9125) (width 0.15) (layer "F.Cu") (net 5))
 (segment (start 125 80) (end 125.0875 80) (width 0.15) (layer "F.Cu") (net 5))
 (segment (start 124 80.9125) (end 124.9125 80) (width 0.15) (layer "F.Cu") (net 5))
 (segment (start 126 79.0875) (end 126.175 79.0875) (width 0.15) (layer "F.Cu") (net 1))
 (segment (start 126 76.6875) (end 126 79.0875) (width 0.15) (layer "F.Cu") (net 1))
 (segment (start 126.175 79.0875) (end 128 80.9125) (width 0.15) (layer "F.Cu") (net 1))
 (segment (start 130 79.0875) (end 128 79.0875) (width 0.15) (layer "F.Cu") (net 2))
 (segment (start 128 78) (end 126.6875 76.6875) (width 0.15) (layer "F.Cu") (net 2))
 (segment (start 128 79.0875) (end 128 78) (width 0.15) (layer "F.Cu") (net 2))
 (segment (start 126.6875 76.6875) (end 126.6875 76) (width 0.15) (layer "F.Cu") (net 2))
 (segment (start 129 77) (end 130.0875 77) (width 0.15) (layer "F.Cu") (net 11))
 (segment (start 130.0875 77.175) (end 132 79.0875) (width 0.15) (layer "F.Cu") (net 11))
 (segment (start 127.5 75.5) (end 129 77) (width 0.15) (layer "F.Cu") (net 11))
 (segment (start 126.6875 75.5) (end 127.5 75.5) (width 0.15) (layer "F.Cu") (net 11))
 (segment (start 130.0875 77) (end 130.0875 77.175) (width 0.15) (layer "F.Cu") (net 11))
 (segment (start 125 73.3125) (end 125 72.5) (width 0.3) (layer "F.Cu") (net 15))
 (via (at 125.5 72) (size 0.6) (drill 0.3) (layers "F.Cu" "B.Cu") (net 15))
 (via (at 125 72.5) (size 0.6) (drill 0.3) (layers "F.Cu" "B.Cu") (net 15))
 (segment (start 130.15 71) (end 130.15 73.7) (width 0.5) (layer "F.Cu") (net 13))
 (segment (start 130.15 73.7) (end 130.45 74) (width 0.5) (layer "F.Cu") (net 13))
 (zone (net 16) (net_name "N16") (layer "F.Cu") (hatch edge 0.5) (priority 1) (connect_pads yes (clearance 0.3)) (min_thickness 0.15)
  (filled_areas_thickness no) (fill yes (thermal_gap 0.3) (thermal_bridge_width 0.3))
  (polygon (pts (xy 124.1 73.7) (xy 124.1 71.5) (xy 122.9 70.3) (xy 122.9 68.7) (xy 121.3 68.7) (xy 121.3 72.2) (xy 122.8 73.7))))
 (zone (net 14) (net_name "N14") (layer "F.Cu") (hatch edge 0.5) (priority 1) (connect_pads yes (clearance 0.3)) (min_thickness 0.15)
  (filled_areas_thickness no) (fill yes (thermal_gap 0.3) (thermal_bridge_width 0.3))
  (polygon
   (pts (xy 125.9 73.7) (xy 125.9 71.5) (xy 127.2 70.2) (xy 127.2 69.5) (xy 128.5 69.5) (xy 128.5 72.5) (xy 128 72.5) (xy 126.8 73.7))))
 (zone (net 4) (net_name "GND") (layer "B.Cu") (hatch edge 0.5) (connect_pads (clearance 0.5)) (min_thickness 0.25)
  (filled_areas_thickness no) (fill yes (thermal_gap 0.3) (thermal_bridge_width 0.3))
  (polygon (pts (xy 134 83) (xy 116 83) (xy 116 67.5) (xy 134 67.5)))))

